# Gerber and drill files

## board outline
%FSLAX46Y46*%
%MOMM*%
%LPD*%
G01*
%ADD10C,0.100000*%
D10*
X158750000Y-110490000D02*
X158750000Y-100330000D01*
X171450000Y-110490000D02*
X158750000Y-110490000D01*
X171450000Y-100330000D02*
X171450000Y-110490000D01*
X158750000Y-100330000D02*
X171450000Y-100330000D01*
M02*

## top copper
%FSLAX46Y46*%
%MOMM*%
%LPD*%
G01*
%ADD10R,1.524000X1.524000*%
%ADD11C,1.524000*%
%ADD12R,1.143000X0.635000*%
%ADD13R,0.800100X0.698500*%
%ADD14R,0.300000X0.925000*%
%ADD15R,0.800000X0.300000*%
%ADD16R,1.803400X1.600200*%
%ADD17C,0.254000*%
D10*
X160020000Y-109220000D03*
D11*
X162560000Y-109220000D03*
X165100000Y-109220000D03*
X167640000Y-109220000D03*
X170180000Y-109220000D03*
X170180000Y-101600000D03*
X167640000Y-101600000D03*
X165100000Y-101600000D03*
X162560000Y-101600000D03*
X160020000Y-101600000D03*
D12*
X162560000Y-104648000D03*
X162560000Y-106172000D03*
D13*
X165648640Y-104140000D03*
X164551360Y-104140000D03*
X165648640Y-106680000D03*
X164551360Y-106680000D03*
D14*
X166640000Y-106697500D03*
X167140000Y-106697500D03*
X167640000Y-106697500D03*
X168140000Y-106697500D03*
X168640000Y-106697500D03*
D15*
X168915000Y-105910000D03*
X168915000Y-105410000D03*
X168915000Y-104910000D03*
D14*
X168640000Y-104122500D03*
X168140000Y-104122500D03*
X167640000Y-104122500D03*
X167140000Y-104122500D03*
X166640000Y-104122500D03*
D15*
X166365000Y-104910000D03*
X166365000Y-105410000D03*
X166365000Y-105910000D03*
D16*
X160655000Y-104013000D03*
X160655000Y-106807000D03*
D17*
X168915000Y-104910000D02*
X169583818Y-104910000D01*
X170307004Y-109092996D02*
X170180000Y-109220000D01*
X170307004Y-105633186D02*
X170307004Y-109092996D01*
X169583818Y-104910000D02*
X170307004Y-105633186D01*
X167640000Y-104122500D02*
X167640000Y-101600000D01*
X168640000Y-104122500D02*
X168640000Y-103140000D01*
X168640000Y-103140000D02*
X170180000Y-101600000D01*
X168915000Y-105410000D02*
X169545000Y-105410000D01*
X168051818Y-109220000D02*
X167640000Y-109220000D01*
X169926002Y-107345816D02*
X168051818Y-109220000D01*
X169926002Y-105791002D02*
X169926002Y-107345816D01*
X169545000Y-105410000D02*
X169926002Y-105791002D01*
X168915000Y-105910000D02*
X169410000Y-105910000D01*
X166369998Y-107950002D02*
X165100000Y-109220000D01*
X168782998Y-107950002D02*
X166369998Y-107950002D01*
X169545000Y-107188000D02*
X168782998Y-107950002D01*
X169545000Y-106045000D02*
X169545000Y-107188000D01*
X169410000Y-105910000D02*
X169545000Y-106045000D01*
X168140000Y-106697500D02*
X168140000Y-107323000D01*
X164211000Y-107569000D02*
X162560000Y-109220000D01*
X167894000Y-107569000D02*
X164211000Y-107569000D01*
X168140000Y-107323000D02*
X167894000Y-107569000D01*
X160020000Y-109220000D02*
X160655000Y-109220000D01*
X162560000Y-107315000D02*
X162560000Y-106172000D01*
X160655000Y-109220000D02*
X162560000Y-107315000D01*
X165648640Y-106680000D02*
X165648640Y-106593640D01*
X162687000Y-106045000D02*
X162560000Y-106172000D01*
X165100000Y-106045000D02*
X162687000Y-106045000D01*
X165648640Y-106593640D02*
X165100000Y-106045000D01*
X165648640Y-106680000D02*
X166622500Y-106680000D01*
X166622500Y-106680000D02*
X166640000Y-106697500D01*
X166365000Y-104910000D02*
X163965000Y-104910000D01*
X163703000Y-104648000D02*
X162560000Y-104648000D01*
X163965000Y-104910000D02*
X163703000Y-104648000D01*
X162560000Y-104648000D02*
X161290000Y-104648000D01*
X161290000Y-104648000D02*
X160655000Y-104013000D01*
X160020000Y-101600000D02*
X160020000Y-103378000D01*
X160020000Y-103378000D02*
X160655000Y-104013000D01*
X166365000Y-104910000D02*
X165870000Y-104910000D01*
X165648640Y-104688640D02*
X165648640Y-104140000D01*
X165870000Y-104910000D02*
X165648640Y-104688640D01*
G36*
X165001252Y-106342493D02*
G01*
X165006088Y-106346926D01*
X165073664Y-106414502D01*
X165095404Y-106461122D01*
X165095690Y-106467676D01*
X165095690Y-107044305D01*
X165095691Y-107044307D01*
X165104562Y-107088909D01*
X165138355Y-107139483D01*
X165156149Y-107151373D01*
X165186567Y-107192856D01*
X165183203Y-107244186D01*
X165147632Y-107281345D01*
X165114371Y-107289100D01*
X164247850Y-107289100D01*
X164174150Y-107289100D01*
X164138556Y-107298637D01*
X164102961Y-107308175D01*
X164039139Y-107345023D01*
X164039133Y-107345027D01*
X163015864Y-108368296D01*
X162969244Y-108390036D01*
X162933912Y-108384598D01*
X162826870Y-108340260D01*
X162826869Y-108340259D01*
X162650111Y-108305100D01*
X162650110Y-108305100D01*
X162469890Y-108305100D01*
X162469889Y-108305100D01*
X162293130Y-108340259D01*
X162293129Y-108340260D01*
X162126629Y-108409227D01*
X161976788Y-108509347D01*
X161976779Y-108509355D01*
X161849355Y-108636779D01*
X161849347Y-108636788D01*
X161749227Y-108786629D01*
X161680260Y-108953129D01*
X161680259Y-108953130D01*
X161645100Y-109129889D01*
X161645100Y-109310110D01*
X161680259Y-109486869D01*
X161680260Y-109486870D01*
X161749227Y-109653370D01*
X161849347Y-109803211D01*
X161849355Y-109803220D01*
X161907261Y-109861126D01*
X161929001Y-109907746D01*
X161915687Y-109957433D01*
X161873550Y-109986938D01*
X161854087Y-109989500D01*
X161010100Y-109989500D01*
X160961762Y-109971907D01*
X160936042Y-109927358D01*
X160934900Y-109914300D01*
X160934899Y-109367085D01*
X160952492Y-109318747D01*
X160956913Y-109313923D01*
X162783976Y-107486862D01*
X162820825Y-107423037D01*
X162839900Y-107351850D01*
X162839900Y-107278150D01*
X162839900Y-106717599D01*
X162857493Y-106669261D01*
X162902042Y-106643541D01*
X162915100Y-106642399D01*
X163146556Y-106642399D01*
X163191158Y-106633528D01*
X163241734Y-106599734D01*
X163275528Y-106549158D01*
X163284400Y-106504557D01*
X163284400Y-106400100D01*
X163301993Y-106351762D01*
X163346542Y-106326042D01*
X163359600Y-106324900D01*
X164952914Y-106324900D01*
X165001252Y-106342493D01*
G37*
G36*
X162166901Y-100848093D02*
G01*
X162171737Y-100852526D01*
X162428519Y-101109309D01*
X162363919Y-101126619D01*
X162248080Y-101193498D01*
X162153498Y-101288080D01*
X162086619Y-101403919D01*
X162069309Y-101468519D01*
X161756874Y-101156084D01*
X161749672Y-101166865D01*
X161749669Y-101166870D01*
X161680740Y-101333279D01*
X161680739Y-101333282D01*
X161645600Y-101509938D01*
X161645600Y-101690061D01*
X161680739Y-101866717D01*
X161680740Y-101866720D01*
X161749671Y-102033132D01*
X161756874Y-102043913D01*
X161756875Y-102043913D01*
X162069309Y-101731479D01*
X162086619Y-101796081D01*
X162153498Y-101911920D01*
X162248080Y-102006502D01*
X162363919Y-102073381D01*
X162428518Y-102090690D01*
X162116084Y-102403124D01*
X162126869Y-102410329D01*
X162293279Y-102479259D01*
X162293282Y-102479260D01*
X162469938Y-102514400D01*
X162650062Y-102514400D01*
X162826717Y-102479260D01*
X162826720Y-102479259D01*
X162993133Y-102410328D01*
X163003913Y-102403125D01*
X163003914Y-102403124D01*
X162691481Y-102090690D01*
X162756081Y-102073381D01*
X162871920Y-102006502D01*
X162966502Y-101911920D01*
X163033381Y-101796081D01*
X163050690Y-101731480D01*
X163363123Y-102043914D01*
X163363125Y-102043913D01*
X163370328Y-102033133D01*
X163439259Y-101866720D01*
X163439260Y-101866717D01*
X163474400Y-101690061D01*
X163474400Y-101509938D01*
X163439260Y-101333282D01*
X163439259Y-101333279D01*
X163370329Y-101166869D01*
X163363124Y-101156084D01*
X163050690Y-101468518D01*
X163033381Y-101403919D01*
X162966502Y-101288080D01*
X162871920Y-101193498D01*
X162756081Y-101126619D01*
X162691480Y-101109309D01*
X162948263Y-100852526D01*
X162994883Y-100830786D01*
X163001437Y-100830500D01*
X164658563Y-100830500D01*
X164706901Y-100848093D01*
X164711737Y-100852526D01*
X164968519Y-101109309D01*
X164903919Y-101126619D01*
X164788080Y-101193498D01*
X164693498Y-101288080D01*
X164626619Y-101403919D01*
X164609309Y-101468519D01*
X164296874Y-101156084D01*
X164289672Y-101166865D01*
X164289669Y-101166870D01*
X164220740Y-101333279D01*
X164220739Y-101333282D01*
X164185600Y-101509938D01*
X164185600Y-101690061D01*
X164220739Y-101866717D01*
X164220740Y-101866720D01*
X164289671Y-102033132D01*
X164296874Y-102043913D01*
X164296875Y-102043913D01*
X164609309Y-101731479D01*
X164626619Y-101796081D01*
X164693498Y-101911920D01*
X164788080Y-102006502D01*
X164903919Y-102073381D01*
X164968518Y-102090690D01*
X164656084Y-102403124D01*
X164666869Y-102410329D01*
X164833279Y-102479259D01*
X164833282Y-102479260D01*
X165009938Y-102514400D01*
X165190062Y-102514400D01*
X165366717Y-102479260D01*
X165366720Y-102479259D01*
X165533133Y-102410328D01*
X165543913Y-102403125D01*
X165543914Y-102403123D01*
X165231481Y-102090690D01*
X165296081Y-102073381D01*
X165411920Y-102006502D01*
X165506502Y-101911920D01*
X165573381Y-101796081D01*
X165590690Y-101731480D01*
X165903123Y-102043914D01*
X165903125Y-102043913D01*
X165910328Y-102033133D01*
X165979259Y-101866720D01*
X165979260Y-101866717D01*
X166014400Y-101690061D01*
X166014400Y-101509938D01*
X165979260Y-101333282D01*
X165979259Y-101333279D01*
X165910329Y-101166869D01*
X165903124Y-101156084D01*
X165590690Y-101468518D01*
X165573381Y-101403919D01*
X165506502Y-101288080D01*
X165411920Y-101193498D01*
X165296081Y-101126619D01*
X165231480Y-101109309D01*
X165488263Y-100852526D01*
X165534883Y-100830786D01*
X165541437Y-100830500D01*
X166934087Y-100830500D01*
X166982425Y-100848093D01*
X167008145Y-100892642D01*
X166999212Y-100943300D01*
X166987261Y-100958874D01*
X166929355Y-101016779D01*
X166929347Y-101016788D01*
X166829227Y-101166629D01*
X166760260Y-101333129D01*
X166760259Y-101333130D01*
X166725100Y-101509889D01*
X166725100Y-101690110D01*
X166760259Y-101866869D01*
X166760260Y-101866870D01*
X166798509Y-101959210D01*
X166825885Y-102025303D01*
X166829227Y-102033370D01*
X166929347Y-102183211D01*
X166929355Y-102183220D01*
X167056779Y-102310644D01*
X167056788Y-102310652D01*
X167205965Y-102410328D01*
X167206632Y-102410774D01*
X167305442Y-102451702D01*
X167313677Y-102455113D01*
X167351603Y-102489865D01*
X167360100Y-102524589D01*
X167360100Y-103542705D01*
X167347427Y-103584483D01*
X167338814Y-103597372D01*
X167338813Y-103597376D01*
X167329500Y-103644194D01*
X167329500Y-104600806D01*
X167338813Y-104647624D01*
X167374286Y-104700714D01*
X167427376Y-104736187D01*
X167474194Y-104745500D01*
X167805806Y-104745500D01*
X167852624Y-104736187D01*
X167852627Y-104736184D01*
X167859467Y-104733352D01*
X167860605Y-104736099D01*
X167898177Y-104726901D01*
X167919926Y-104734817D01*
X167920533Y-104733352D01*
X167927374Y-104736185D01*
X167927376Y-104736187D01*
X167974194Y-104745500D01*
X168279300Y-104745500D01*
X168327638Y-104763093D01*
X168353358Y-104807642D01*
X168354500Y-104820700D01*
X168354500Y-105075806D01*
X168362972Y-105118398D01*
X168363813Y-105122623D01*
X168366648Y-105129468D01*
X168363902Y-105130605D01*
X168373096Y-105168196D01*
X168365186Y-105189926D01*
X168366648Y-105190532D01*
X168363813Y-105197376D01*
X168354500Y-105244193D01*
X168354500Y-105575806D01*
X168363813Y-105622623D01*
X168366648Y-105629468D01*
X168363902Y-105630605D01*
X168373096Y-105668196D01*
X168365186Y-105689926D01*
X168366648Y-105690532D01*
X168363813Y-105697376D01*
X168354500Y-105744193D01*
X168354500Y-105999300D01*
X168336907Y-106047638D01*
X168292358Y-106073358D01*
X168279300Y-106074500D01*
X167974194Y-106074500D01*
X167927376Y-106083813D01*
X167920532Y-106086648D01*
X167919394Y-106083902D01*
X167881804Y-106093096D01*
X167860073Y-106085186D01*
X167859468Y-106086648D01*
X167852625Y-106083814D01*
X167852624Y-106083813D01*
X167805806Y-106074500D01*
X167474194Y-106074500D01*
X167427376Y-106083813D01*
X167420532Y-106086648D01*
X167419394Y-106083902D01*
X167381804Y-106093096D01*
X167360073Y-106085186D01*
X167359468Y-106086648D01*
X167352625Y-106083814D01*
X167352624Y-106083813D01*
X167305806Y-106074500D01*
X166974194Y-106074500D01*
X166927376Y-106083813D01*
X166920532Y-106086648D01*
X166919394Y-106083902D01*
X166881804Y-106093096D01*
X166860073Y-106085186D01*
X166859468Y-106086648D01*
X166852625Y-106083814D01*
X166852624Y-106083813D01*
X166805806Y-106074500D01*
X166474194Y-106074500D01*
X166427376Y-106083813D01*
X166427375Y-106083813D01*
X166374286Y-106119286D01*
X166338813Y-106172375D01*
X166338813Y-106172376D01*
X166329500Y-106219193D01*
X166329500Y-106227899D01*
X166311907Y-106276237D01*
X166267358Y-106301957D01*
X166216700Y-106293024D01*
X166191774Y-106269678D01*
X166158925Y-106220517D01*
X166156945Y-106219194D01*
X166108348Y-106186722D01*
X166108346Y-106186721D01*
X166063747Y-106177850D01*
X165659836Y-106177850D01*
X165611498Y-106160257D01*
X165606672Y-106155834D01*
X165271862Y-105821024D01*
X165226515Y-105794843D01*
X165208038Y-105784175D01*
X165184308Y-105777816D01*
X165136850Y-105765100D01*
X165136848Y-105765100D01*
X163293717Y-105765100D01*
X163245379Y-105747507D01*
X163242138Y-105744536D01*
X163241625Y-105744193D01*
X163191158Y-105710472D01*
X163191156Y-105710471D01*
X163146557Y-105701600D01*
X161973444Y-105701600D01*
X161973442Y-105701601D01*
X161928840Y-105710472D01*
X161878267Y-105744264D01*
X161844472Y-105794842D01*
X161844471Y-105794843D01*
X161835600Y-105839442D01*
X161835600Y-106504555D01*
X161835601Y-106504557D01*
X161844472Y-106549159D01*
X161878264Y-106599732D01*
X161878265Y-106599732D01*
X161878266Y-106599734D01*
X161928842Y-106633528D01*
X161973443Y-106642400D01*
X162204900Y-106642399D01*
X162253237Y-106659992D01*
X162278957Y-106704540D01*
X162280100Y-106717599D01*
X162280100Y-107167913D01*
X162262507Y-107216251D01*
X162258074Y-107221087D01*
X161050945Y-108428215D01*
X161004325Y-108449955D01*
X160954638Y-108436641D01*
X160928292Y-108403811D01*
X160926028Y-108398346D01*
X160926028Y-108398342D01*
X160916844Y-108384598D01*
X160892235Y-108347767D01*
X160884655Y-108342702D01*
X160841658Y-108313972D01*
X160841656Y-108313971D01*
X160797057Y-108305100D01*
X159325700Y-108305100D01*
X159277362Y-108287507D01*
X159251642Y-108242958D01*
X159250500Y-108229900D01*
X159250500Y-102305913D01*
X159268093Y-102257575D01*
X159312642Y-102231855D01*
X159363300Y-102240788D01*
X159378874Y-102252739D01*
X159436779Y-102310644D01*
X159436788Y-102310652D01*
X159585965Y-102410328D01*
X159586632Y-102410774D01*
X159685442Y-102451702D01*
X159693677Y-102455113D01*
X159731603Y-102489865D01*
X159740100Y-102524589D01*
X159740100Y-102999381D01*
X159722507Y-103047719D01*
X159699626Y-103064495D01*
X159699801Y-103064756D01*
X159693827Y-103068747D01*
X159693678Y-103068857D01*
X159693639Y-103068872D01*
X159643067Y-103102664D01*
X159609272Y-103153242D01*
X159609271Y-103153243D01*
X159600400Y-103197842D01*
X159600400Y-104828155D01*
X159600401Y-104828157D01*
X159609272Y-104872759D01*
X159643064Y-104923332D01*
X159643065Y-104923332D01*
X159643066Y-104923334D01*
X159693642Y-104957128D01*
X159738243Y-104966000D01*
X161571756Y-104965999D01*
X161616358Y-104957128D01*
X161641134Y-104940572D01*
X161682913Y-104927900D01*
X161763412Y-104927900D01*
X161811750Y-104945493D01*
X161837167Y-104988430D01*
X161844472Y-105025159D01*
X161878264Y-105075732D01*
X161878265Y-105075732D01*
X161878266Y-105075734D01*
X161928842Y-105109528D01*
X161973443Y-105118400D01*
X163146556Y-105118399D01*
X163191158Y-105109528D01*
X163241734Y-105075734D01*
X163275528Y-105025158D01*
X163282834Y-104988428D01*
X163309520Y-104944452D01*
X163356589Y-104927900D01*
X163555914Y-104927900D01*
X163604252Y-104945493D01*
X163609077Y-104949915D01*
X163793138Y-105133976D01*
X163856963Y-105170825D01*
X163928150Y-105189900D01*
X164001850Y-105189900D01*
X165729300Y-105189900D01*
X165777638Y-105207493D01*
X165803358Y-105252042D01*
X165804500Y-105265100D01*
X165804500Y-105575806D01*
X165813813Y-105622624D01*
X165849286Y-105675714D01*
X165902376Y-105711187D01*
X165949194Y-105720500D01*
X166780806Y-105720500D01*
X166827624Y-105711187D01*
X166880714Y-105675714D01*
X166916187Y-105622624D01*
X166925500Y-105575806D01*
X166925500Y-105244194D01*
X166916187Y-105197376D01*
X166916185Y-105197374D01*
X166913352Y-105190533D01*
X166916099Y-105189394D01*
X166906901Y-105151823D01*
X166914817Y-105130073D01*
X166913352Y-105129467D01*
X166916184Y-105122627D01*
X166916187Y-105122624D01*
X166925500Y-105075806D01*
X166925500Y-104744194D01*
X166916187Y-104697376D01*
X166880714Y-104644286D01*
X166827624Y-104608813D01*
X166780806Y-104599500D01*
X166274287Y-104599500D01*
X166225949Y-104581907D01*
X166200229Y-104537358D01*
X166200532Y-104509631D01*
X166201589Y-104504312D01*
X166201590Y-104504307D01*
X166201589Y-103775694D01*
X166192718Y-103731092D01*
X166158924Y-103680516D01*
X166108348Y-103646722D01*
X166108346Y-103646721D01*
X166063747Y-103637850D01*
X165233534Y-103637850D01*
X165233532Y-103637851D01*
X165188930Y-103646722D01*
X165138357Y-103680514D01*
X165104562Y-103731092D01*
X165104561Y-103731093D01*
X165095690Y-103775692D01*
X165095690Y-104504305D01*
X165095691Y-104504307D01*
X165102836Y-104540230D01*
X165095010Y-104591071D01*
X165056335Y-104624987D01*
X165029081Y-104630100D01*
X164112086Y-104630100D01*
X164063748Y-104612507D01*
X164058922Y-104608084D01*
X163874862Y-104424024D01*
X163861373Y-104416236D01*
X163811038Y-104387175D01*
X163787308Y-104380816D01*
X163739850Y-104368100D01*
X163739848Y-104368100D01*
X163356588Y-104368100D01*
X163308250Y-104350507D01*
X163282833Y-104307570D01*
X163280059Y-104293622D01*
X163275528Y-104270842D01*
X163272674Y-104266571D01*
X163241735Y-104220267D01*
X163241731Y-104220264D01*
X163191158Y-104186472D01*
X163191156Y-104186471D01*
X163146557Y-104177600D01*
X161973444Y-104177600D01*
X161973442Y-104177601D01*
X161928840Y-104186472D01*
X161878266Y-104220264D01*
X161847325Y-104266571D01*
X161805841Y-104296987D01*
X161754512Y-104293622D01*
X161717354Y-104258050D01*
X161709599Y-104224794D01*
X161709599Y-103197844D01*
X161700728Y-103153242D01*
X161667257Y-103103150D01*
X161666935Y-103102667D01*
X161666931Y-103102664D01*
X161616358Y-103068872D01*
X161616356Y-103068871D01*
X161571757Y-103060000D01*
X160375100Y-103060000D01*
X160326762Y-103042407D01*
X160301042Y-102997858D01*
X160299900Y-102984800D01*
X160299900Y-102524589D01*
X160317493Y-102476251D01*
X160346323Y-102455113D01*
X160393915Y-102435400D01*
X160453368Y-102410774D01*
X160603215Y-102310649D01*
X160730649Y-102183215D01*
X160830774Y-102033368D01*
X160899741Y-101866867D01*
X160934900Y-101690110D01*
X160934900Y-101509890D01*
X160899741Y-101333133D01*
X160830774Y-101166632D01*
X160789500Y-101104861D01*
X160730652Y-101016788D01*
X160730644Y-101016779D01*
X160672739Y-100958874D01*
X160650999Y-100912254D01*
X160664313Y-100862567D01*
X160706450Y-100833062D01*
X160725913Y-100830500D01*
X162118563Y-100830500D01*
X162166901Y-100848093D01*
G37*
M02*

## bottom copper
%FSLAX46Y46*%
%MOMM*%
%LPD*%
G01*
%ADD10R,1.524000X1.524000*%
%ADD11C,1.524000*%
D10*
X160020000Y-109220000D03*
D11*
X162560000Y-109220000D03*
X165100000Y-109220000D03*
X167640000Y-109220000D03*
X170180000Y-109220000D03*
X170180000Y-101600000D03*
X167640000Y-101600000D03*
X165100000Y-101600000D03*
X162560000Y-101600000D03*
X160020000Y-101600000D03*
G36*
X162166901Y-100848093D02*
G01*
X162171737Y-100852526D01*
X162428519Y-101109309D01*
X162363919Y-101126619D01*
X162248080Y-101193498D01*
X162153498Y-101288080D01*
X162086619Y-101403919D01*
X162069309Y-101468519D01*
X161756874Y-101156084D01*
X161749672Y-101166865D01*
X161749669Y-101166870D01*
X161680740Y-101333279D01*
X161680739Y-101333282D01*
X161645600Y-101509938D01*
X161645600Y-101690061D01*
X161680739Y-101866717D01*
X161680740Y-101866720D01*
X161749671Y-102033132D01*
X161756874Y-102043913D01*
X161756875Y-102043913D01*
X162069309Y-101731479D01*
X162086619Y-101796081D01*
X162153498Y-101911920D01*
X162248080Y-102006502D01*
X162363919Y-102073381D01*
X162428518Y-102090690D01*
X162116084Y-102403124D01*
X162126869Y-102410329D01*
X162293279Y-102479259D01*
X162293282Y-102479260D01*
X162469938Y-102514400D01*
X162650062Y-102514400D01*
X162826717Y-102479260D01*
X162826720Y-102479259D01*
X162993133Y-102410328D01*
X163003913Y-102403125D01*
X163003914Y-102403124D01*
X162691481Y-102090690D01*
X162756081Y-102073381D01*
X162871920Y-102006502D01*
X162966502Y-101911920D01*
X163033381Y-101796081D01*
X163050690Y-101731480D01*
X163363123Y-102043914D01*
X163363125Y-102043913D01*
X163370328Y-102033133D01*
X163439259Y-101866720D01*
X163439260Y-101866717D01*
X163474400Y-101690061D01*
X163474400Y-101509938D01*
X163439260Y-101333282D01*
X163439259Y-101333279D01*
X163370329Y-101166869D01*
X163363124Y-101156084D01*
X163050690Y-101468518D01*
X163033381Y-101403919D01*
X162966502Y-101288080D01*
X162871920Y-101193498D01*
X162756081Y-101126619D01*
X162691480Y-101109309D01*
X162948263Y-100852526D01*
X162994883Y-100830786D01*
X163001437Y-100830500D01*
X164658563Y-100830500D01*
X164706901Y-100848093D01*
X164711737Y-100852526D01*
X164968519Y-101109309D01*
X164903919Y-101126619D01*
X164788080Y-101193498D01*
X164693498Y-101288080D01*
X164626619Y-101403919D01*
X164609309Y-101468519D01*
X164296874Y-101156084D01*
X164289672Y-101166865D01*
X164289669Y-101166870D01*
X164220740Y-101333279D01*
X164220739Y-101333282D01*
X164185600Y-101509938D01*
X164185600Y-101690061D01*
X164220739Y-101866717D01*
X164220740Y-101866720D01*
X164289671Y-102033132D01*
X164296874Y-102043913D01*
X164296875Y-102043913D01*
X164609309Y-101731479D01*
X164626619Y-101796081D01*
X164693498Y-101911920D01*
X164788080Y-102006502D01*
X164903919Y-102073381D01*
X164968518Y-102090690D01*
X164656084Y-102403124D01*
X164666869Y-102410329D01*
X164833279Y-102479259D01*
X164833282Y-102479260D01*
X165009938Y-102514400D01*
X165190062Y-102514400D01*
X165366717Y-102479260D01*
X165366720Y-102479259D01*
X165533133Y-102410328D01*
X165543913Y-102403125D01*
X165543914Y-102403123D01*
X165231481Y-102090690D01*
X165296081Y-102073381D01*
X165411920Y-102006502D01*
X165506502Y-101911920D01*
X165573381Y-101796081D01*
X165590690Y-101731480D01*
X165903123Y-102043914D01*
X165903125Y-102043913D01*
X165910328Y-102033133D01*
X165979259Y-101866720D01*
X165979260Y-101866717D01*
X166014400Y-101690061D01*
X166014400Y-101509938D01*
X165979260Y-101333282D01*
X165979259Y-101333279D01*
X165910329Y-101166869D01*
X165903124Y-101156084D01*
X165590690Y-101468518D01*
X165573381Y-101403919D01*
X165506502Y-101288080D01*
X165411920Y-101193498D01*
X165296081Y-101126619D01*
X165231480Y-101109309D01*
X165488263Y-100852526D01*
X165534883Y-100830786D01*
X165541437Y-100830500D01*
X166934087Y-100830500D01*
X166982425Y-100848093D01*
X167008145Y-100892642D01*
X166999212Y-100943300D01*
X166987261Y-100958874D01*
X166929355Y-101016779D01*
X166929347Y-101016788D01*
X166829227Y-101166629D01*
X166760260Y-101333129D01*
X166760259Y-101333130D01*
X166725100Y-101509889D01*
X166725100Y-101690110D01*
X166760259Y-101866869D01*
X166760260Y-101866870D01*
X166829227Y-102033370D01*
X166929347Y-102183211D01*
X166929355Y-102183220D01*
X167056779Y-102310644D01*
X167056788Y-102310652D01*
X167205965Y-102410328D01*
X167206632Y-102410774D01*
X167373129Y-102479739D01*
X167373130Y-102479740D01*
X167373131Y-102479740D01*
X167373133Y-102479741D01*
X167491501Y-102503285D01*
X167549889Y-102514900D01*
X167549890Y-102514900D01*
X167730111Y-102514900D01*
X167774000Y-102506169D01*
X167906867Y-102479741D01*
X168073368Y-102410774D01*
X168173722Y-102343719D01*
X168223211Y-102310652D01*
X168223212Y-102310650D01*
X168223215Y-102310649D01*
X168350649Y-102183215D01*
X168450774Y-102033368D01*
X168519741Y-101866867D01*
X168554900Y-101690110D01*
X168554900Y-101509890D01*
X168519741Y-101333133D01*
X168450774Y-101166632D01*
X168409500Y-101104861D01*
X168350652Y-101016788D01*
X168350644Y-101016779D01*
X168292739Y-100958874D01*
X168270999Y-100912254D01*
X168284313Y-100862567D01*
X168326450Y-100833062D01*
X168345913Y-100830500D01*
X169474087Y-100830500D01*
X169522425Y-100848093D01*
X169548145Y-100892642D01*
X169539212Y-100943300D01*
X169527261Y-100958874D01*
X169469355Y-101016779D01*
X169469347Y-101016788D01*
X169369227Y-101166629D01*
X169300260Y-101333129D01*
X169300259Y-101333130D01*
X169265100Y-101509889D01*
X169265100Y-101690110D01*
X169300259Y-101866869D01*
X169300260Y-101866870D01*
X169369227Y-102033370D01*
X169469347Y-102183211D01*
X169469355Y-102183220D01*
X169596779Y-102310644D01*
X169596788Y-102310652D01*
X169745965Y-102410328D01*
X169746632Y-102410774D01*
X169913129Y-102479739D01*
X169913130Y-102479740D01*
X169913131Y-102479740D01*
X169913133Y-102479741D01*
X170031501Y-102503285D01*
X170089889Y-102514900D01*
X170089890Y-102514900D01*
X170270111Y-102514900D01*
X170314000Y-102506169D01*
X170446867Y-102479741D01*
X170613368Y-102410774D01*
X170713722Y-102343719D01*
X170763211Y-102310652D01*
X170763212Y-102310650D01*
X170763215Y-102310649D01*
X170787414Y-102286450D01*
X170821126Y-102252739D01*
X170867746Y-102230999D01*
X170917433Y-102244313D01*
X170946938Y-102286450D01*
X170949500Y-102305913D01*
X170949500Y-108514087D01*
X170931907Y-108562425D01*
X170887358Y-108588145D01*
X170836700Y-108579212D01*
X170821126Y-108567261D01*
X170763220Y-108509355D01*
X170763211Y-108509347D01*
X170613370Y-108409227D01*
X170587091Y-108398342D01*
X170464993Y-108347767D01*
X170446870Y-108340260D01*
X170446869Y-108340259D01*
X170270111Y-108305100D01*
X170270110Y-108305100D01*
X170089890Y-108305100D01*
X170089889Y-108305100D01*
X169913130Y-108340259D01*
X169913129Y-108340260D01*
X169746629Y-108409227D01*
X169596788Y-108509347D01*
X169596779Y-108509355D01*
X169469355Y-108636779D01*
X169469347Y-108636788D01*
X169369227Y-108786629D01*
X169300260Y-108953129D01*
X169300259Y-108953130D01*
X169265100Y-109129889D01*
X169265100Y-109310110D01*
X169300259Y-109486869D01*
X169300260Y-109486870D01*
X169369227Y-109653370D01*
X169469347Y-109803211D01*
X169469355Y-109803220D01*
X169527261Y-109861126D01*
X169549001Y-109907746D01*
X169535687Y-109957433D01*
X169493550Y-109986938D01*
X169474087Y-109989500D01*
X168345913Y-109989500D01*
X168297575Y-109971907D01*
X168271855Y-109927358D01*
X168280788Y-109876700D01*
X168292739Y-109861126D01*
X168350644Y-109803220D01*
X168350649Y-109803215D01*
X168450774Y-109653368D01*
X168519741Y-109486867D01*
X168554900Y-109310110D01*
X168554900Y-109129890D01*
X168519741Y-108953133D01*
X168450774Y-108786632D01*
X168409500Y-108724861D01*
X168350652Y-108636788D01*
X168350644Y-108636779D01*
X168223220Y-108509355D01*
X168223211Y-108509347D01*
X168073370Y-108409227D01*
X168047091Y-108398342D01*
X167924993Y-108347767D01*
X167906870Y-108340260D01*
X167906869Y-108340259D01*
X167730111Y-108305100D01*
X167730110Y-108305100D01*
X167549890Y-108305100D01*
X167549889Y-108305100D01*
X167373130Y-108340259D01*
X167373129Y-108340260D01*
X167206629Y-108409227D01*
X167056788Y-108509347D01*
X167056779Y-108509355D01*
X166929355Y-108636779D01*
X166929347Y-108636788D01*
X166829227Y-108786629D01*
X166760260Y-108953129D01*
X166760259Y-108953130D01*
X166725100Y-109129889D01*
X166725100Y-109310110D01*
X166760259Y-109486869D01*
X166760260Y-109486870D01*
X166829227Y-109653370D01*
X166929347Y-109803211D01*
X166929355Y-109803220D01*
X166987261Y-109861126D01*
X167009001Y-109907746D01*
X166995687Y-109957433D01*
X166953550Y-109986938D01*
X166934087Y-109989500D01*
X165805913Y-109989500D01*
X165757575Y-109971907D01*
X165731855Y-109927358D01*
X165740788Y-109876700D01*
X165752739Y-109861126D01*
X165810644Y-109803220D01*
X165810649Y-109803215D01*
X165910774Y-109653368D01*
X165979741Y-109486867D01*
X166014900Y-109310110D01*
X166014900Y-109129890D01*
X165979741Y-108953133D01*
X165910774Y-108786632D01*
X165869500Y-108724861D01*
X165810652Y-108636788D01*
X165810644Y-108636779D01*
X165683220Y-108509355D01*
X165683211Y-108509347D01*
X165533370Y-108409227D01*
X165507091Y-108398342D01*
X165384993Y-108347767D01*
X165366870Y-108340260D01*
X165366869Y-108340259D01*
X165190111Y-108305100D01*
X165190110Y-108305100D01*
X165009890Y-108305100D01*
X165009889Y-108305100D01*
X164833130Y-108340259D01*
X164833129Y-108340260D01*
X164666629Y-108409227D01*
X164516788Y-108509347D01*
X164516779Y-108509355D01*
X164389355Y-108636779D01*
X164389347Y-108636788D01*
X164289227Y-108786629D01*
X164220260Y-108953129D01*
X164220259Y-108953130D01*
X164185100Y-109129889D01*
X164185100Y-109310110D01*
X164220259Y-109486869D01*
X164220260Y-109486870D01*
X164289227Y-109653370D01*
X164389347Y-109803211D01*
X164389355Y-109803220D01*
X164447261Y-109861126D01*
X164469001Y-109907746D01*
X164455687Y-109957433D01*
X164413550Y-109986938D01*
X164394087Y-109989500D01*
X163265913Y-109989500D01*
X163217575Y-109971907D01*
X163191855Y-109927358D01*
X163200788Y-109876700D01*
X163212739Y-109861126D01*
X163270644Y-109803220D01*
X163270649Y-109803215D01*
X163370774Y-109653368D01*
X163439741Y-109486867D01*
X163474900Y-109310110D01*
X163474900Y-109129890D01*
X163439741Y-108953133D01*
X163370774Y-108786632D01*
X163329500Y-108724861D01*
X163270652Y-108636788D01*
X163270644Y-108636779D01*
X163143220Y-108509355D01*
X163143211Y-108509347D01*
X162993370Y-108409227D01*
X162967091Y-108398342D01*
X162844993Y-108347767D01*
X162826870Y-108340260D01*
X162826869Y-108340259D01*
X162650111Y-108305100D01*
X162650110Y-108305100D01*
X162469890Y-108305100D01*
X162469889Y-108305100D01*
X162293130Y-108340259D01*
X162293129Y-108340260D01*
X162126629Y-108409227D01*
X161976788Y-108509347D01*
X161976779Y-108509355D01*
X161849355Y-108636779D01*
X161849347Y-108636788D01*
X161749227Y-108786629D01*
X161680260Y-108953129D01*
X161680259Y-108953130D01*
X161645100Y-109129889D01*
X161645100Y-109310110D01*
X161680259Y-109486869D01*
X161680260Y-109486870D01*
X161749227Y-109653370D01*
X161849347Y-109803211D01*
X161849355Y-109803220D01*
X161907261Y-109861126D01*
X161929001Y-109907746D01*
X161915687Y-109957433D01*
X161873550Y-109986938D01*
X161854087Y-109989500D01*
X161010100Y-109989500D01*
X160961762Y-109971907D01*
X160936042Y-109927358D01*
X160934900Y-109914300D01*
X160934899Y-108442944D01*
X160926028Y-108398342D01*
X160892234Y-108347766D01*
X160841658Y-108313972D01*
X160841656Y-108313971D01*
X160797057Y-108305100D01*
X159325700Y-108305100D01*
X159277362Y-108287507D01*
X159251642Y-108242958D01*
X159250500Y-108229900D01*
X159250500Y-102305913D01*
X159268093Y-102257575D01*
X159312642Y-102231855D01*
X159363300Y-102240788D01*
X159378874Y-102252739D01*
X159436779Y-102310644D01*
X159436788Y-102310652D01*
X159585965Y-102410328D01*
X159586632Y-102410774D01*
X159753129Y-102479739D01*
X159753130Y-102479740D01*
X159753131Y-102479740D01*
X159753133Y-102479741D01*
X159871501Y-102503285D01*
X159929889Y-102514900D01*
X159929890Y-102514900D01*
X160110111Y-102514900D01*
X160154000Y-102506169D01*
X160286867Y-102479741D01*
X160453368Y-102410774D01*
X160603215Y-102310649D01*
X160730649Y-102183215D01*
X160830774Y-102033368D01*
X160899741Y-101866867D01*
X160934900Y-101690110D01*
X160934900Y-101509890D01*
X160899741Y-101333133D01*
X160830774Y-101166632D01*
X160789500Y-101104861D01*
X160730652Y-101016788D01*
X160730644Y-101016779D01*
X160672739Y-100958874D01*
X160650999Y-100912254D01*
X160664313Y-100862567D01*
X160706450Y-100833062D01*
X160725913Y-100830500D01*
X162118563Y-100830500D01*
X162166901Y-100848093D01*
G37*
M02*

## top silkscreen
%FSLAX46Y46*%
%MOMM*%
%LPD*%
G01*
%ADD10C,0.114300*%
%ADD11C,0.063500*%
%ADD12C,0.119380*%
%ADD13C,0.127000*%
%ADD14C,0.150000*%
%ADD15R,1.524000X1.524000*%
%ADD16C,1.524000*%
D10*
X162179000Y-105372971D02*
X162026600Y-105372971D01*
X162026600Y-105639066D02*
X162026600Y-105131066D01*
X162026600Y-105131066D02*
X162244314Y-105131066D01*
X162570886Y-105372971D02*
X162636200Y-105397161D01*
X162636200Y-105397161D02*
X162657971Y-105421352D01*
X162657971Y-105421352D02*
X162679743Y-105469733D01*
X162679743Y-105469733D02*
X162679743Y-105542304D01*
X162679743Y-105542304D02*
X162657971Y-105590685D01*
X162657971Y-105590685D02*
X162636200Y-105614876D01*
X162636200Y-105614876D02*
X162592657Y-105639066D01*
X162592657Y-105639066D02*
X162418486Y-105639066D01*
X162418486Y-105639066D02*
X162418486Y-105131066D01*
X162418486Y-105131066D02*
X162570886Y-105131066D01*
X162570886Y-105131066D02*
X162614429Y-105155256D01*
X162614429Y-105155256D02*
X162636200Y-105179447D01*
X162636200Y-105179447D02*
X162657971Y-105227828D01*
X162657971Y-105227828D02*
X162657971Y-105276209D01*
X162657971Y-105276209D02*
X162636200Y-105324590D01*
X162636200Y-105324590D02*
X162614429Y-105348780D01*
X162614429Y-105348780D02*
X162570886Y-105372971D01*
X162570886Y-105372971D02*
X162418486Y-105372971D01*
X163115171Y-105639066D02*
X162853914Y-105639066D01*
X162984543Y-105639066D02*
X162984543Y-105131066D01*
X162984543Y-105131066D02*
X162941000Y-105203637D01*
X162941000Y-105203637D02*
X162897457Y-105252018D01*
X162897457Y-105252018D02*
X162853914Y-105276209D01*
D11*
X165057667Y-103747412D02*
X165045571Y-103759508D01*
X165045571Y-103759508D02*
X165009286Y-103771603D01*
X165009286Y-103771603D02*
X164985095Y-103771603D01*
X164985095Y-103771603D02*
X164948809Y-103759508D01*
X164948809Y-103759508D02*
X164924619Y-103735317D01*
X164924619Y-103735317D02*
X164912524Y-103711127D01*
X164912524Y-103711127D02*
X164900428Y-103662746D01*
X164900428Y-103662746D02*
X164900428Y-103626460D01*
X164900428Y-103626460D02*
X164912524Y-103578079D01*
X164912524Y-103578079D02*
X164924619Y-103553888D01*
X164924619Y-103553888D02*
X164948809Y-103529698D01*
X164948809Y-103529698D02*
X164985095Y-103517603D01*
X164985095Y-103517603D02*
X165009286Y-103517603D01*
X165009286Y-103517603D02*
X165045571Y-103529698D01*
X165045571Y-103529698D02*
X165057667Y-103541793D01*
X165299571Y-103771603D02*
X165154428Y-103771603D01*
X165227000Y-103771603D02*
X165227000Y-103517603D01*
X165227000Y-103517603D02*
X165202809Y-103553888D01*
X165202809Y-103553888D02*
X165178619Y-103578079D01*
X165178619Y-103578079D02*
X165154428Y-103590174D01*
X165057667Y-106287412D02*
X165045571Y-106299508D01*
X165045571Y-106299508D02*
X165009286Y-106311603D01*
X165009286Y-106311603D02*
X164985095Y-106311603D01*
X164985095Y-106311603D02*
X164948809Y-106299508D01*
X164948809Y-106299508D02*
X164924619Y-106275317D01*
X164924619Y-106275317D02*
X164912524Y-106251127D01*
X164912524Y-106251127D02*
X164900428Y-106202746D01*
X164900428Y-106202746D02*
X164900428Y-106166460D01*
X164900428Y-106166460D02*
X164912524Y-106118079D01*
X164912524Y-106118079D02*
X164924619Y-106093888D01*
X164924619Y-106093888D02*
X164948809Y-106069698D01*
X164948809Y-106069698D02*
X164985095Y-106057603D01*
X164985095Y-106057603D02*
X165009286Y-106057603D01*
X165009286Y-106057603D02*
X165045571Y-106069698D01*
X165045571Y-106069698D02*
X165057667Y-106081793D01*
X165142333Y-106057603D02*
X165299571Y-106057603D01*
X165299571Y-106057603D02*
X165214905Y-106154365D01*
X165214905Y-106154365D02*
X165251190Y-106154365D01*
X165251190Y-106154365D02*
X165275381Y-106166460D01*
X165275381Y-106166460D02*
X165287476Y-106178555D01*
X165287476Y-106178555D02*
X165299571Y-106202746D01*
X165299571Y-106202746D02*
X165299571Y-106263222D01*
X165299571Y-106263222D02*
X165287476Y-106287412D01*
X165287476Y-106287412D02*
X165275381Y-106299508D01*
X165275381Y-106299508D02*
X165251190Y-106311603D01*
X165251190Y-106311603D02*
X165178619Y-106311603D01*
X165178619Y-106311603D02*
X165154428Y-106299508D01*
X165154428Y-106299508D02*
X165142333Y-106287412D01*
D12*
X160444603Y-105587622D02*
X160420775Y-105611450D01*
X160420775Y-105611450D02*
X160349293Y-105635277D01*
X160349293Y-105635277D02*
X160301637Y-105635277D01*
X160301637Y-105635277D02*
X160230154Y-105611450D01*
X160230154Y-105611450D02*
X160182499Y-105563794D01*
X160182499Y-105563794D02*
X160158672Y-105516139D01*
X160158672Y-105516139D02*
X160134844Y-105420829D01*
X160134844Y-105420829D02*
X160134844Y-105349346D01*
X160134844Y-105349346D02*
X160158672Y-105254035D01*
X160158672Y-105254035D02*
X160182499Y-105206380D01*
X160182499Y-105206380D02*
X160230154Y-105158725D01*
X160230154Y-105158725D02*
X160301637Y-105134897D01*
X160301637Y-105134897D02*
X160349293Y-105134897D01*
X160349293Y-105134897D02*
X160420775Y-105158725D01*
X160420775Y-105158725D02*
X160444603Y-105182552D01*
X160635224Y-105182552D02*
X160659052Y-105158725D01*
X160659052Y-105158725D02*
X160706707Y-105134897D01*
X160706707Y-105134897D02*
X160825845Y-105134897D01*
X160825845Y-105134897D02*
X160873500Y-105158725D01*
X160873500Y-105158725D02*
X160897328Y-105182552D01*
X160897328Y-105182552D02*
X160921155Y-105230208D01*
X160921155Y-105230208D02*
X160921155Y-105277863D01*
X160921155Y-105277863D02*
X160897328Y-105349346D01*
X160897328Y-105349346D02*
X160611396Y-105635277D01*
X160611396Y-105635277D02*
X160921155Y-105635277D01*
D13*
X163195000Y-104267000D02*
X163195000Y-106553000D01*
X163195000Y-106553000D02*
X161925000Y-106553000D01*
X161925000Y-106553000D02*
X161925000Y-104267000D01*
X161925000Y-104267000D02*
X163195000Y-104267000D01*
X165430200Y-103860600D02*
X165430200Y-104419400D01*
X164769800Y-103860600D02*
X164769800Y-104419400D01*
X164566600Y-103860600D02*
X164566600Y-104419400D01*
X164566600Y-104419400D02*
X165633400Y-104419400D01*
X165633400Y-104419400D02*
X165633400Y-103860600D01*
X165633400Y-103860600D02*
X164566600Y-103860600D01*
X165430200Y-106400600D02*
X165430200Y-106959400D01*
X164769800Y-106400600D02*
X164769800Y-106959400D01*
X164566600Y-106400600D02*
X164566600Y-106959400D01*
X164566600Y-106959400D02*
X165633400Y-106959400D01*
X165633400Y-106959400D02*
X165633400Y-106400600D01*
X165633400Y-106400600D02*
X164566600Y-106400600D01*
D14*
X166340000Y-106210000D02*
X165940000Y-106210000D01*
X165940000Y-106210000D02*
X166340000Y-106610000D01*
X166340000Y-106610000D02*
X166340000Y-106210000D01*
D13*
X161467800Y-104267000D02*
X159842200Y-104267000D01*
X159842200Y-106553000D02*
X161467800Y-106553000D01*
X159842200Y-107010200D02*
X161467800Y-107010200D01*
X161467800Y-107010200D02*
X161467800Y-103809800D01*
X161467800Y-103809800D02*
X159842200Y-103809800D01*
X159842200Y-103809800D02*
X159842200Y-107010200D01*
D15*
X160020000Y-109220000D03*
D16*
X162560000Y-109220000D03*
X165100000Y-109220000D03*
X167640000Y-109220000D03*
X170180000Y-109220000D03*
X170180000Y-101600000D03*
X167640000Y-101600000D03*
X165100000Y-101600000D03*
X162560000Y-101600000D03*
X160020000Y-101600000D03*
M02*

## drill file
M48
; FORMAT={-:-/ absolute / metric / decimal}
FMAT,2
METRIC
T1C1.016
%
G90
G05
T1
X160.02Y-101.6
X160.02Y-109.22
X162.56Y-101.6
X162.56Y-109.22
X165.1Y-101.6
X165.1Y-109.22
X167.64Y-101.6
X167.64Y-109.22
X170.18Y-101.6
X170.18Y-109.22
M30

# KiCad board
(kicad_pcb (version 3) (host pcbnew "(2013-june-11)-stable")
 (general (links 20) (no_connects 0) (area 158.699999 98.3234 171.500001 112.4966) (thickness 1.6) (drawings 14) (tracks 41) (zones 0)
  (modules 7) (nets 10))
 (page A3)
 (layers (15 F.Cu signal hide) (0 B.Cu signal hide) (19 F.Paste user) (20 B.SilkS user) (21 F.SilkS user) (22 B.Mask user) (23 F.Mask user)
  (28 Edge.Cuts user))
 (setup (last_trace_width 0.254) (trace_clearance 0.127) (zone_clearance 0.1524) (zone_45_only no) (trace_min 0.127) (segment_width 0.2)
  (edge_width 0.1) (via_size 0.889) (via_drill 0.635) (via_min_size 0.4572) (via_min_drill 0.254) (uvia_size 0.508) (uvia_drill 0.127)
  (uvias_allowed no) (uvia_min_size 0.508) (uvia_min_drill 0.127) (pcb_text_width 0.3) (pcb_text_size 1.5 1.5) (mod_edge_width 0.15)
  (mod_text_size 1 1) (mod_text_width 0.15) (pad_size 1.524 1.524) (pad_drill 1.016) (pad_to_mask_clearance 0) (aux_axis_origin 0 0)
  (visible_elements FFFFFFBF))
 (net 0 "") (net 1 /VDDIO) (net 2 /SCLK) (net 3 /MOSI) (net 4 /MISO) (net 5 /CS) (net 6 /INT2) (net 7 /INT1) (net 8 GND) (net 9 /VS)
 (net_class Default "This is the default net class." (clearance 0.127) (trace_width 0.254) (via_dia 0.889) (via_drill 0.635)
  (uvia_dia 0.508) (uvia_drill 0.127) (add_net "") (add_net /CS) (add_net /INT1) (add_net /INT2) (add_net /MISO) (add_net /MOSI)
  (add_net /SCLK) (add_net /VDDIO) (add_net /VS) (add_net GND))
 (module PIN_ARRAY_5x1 (layer F.Cu) (at 165.1 109.22)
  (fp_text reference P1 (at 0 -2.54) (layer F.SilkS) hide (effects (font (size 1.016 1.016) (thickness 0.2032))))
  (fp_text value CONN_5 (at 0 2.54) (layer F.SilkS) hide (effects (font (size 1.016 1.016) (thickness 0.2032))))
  (pad 1 thru_hole rect (at -5.08 0) (size 1.524 1.524) (drill 1.016) (layers *.Cu *.Mask F.SilkS) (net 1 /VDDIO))
  (pad 2 thru_hole circle (at -2.54 0) (size 1.524 1.524) (drill 1.016) (layers *.Cu *.Mask F.SilkS) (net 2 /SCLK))
  (pad 3 thru_hole circle (at 0 0) (size 1.524 1.524) (drill 1.016) (layers *.Cu *.Mask F.SilkS) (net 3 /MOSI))
  (pad 4 thru_hole circle (at 2.54 0) (size 1.524 1.524) (drill 1.016) (layers *.Cu *.Mask F.SilkS) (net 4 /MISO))
  (pad 5 thru_hole circle (at 5.08 0) (size 1.524 1.524) (drill 1.016) (layers *.Cu *.Mask F.SilkS) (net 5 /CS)))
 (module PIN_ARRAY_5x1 (layer F.Cu) (at 165.1 101.6 180)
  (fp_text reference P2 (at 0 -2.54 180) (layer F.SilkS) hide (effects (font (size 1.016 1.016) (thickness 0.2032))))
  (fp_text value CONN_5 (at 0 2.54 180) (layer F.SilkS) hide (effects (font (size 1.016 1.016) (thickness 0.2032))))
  (pad 1 thru_hole circle (at -5.08 0 180) (size 1.524 1.524) (drill 1.016) (layers *.Cu *.Mask F.SilkS) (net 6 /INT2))
  (pad 2 thru_hole circle (at -2.54 0 180) (size 1.524 1.524) (drill 1.016) (layers *.Cu *.Mask F.SilkS) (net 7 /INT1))
  (pad 3 thru_hole circle (at 0 0 180) (size 1.524 1.524) (drill 1.016) (layers *.Cu *.Mask F.SilkS) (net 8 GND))
  (pad 4 thru_hole circle (at 2.54 0 180) (size 1.524 1.524) (drill 1.016) (layers *.Cu *.Mask F.SilkS) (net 8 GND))
  (pad 5 thru_hole circle (at 5.08 0 180) (size 1.524 1.524) (drill 1.016) (layers *.Cu *.Mask F.SilkS) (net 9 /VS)))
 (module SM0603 (layer F.Cu) (at 162.56 105.41 270)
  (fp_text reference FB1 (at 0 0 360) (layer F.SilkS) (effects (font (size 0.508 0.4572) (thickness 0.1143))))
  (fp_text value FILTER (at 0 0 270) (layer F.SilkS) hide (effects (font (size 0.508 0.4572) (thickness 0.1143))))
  (fp_line (start -1.143 -0.635) (end 1.143 -0.635) (layer F.SilkS) (width 0.127))
  (fp_line (start 1.143 -0.635) (end 1.143 0.635) (layer F.SilkS) (width 0.127))
  (fp_line (start 1.143 0.635) (end -1.143 0.635) (layer F.SilkS) (width 0.127))
  (fp_line (start -1.143 0.635) (end -1.143 -0.635) (layer F.SilkS) (width 0.127))
  (pad 1 smd rect (at -0.762 0 270) (size 0.635 1.143) (layers F.Cu F.Paste F.Mask) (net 9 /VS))
  (pad 2 smd rect (at 0.762 0 270) (size 0.635 1.143) (layers F.Cu F.Paste F.Mask) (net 1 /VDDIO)))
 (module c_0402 (layer F.Cu) (at 165.1 104.14)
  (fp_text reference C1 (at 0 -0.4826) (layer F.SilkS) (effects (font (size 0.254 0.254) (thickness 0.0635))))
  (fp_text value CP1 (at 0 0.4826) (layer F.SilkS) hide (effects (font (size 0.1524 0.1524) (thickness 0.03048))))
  (fp_line (start 0.3302 -0.2794) (end 0.3302 0.2794) (layer F.SilkS) (width 0.127))
  (fp_line (start -0.3302 -0.2794) (end -0.3302 0.2794) (layer F.SilkS) (width 0.127))
  (fp_line (start -0.5334 -0.2794) (end -0.5334 0.2794) (layer F.SilkS) (width 0.127))
  (fp_line (start -0.5334 0.2794) (end 0.5334 0.2794) (layer F.SilkS) (width 0.127))
  (fp_line (start 0.5334 0.2794) (end 0.5334 -0.2794) (layer F.SilkS) (width 0.127))
  (fp_line (start 0.5334 -0.2794) (end -0.5334 -0.2794) (layer F.SilkS) (width 0.127))
  (pad 1 smd rect (at 0.54864 0) (size 0.8001 0.6985) (layers F.Cu F.Paste F.Mask) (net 9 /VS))
  (pad 2 smd rect (at -0.54864 0) (size 0.8001 0.6985) (layers F.Cu F.Paste F.Mask) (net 8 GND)))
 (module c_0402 (layer F.Cu) (at 165.1 106.68)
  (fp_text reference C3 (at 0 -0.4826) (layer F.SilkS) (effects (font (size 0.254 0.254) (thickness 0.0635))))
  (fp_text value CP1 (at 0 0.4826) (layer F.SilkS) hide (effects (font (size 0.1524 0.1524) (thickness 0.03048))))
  (fp_line (start 0.3302 -0.2794) (end 0.3302 0.2794) (layer F.SilkS) (width 0.127))
  (fp_line (start -0.3302 -0.2794) (end -0.3302 0.2794) (layer F.SilkS) (width 0.127))
  (fp_line (start -0.5334 -0.2794) (end -0.5334 0.2794) (layer F.SilkS) (width 0.127))
  (fp_line (start -0.5334 0.2794) (end 0.5334 0.2794) (layer F.SilkS) (width 0.127))
  (fp_line (start 0.5334 0.2794) (end 0.5334 -0.2794) (layer F.SilkS) (width 0.127))
  (fp_line (start 0.5334 -0.2794) (end -0.5334 -0.2794) (layer F.SilkS) (width 0.127))
  (pad 1 smd rect (at 0.54864 0) (size 0.8001 0.6985) (layers F.Cu F.Paste F.Mask) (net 1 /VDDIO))
  (pad 2 smd rect (at -0.54864 0) (size 0.8001 0.6985) (layers F.Cu F.Paste F.Mask) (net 8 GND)))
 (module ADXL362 (layer F.Cu) (at 167.64 105.41 90) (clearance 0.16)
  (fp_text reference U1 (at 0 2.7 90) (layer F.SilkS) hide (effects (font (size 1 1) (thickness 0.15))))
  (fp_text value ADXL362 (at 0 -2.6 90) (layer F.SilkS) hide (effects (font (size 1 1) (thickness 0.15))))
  (fp_line (start -0.8 -1.3) (end -0.8 -1.7) (layer F.SilkS) (width 0.15))
  (fp_line (start -0.8 -1.7) (end -1.2 -1.3) (layer F.SilkS) (width 0.15))
  (fp_line (start -1.2 -1.3) (end -0.8 -1.3) (layer F.SilkS) (width 0.15))
  (pad 1 smd rect (at -1.2875 -1 90) (size 0.925 0.3) (layers F.Cu F.Paste F.Mask) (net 1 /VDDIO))
  (pad 2 smd rect (at -1.2875 -0.5 90) (size 0.925 0.3) (layers F.Cu F.Paste F.Mask))
  (pad 3 smd rect (at -1.2875 0 90) (size 0.925 0.3) (layers F.Cu F.Paste F.Mask))
  (pad 4 smd rect (at -1.2875 0.5 90) (size 0.925 0.3) (layers F.Cu F.Paste F.Mask) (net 2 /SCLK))
  (pad 5 smd rect (at -1.2875 1 90) (size 0.925 0.3) (layers F.Cu F.Paste F.Mask))
  (pad 6 smd rect (at -0.5 1.275 90) (size 0.3 0.8) (layers F.Cu F.Paste F.Mask) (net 3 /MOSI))
  (pad 7 smd rect (at 0 1.275 90) (size 0.3 0.8) (layers F.Cu F.Paste F.Mask) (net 4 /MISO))
  (pad 8 smd rect (at 0.5 1.275 90) (size 0.3 0.8) (layers F.Cu F.Paste F.Mask) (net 5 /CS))
  (pad 9 smd rect (at 1.2875 1 90) (size 0.925 0.3) (layers F.Cu F.Paste F.Mask) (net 6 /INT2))
  (pad 10 smd rect (at 1.2875 0.5 90) (size 0.925 0.3) (layers F.Cu F.Paste F.Mask))
  (pad 11 smd rect (at 1.2875 0 90) (size 0.925 0.3) (layers F.Cu F.Paste F.Mask) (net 7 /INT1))
  (pad 12 smd rect (at 1.2875 -0.5 90) (size 0.925 0.3) (layers F.Cu F.Paste F.Mask) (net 8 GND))
  (pad 13 smd rect (at 1.2875 -1 90) (size 0.925 0.3) (layers F.Cu F.Paste F.Mask) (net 8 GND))
  (pad 14 smd rect (at 0.5 -1.275 90) (size 0.3 0.8) (layers F.Cu F.Paste F.Mask) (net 9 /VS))
  (pad 15 smd rect (at 0 -1.275 90) (size 0.3 0.8) (layers F.Cu F.Paste F.Mask))
  (pad 16 smd rect (at -0.5 -1.275 90) (size 0.3 0.8) (layers F.Cu F.Paste F.Mask) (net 8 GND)))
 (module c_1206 (layer F.Cu) (at 160.655 105.41 90)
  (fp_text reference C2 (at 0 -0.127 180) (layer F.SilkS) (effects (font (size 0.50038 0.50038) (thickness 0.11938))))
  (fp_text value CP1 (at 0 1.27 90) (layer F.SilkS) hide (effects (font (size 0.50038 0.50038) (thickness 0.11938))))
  (fp_line (start 1.143 0.8128) (end 1.143 -0.8128) (layer F.SilkS) (width 0.127))
  (fp_line (start -1.143 -0.8128) (end -1.143 0.8128) (layer F.SilkS) (width 0.127))
  (fp_line (start -1.6002 -0.8128) (end -1.6002 0.8128) (layer F.SilkS) (width 0.127))
  (fp_line (start -1.6002 0.8128) (end 1.6002 0.8128) (layer F.SilkS) (width 0.127))
  (fp_line (start 1.6002 0.8128) (end 1.6002 -0.8128) (layer F.SilkS) (width 0.127))
  (fp_line (start 1.6002 -0.8128) (end -1.6002 -0.8128) (layer F.SilkS) (width 0.127))
  (pad 1 smd rect (at 1.397 0 90) (size 1.6002 1.8034) (layers F.Cu F.Paste F.Mask) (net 9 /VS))
  (pad 2 smd rect (at -1.397 0 90) (size 1.6002 1.8034) (layers F.Cu F.Paste F.Mask) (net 8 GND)))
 (gr_line (start 158.75 110.49) (end 158.75 100.33) (angle 90) (layer Edge.Cuts) (width 0.1))
 (gr_line (start 171.45 110.49) (end 158.75 110.49) (angle 90) (layer Edge.Cuts) (width 0.1))
 (gr_line (start 171.45 100.33) (end 171.45 110.49) (angle 90) (layer Edge.Cuts) (width 0.1))
 (gr_line (start 158.75 100.33) (end 171.45 100.33) (angle 90) (layer Edge.Cuts) (width 0.1))
 (segment (start 168.915 104.91) (end 169.583818 104.91) (width 0.254) (layer F.Cu) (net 5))
 (segment (start 170.307004 109.092996) (end 170.18 109.22) (width 0.254) (layer F.Cu) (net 5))
 (segment (start 170.307004 105.633186) (end 170.307004 109.092996) (width 0.254) (layer F.Cu) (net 5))
 (segment (start 169.583818 104.91) (end 170.307004 105.633186) (width 0.254) (layer F.Cu) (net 5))
 (segment (start 167.64 104.1225) (end 167.64 101.6) (width 0.254) (layer F.Cu) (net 7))
 (segment (start 168.64 104.1225) (end 168.64 103.14) (width 0.254) (layer F.Cu) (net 6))
 (segment (start 168.64 103.14) (end 170.18 101.6) (width 0.254) (layer F.Cu) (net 6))
 (segment (start 168.915 105.41) (end 169.545 105.41) (width 0.254) (layer F.Cu) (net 4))
 (segment (start 168.051818 109.22) (end 167.64 109.22) (width 0.254) (layer F.Cu) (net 4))
 (segment (start 169.926002 107.345816) (end 168.051818 109.22) (width 0.254) (layer F.Cu) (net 4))
 (segment (start 169.926002 105.791002) (end 169.926002 107.345816) (width 0.254) (layer F.Cu) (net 4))
 (segment (start 169.545 105.41) (end 169.926002 105.791002) (width 0.254) (layer F.Cu) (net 4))
 (segment (start 168.915 105.91) (end 169.41 105.91) (width 0.254) (layer F.Cu) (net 3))
 (segment (start 166.369998 107.950002) (end 165.1 109.22) (width 0.254) (layer F.Cu) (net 3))
 (segment (start 168.782998 107.950002) (end 166.369998 107.950002) (width 0.254) (layer F.Cu) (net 3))
 (segment (start 169.545 107.188) (end 168.782998 107.950002) (width 0.254) (layer F.Cu) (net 3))
 (segment (start 169.545 106.045) (end 169.545 107.188) (width 0.254) (layer F.Cu) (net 3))
 (segment (start 169.41 105.91) (end 169.545 106.045) (width 0.254) (layer F.Cu) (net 3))
 (segment (start 168.14 106.6975) (end 168.14 107.323) (width 0.254) (layer F.Cu) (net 2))
 (segment (start 164.211 107.569) (end 162.56 109.22) (width 0.254) (layer F.Cu) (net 2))
 (segment (start 167.894 107.569) (end 164.211 107.569) (width 0.254) (layer F.Cu) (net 2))
 (segment (start 168.14 107.323) (end 167.894 107.569) (width 0.254) (layer F.Cu) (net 2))
 (segment (start 160.02 109.22) (end 160.655 109.22) (width 0.254) (layer F.Cu) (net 1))
 (segment (start 162.56 107.315) (end 162.56 106.172) (width 0.254) (layer F.Cu) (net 1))
 (segment (start 160.655 109.22) (end 162.56 107.315) (width 0.254) (layer F.Cu) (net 1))
 (segment (start 165.64864 106.68) (end 165.64864 106.59364) (width 0.254) (layer F.Cu) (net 1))
 (segment (start 162.687 106.045) (end 162.56 106.172) (width 0.254) (layer F.Cu) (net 1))
 (segment (start 165.1 106.045) (end 162.687 106.045) (width 0.254) (layer F.Cu) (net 1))
 (segment (start 165.64864 106.59364) (end 165.1 106.045) (width 0.254) (layer F.Cu) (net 1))
 (segment (start 165.64864 106.68) (end 166.6225 106.68) (width 0.254) (layer F.Cu) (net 1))
 (segment (start 166.6225 106.68) (end 166.64 106.6975) (width 0.254) (layer F.Cu) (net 1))
 (segment (start 166.365 104.91) (end 163.965 104.91) (width 0.254) (layer F.Cu) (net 9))
 (segment (start 163.703 104.648) (end 162.56 104.648) (width 0.254) (layer F.Cu) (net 9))
 (segment (start 163.965 104.91) (end 163.703 104.648) (width 0.254) (layer F.Cu) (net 9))
 (segment (start 162.56 104.648) (end 161.29 104.648) (width 0.254) (layer F.Cu) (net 9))
 (segment (start 161.29 104.648) (end 160.655 104.013) (width 0.254) (layer F.Cu) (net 9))
 (segment (start 160.02 101.6) (end 160.02 103.378) (width 0.254) (layer F.Cu) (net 9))
 (segment (start 160.02 103.378) (end 160.655 104.013) (width 0.254) (layer F.Cu) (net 9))
 (segment (start 166.365 104.91) (end 165.87 104.91) (width 0.254) (layer F.Cu) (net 9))
 (segment (start 165.64864 104.68864) (end 165.64864 104.14) (width 0.254) (layer F.Cu) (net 9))
 (segment (start 165.87 104.91) (end 165.64864 104.68864) (width 0.254) (layer F.Cu) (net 9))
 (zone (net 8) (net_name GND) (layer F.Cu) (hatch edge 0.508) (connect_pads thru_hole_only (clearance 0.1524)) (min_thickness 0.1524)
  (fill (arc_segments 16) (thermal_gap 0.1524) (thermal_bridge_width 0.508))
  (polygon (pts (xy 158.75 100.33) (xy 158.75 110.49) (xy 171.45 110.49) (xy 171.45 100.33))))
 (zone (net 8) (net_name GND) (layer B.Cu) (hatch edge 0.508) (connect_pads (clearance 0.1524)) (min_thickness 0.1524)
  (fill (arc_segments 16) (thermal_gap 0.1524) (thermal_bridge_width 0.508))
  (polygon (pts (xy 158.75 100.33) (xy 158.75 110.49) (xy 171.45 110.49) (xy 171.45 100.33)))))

